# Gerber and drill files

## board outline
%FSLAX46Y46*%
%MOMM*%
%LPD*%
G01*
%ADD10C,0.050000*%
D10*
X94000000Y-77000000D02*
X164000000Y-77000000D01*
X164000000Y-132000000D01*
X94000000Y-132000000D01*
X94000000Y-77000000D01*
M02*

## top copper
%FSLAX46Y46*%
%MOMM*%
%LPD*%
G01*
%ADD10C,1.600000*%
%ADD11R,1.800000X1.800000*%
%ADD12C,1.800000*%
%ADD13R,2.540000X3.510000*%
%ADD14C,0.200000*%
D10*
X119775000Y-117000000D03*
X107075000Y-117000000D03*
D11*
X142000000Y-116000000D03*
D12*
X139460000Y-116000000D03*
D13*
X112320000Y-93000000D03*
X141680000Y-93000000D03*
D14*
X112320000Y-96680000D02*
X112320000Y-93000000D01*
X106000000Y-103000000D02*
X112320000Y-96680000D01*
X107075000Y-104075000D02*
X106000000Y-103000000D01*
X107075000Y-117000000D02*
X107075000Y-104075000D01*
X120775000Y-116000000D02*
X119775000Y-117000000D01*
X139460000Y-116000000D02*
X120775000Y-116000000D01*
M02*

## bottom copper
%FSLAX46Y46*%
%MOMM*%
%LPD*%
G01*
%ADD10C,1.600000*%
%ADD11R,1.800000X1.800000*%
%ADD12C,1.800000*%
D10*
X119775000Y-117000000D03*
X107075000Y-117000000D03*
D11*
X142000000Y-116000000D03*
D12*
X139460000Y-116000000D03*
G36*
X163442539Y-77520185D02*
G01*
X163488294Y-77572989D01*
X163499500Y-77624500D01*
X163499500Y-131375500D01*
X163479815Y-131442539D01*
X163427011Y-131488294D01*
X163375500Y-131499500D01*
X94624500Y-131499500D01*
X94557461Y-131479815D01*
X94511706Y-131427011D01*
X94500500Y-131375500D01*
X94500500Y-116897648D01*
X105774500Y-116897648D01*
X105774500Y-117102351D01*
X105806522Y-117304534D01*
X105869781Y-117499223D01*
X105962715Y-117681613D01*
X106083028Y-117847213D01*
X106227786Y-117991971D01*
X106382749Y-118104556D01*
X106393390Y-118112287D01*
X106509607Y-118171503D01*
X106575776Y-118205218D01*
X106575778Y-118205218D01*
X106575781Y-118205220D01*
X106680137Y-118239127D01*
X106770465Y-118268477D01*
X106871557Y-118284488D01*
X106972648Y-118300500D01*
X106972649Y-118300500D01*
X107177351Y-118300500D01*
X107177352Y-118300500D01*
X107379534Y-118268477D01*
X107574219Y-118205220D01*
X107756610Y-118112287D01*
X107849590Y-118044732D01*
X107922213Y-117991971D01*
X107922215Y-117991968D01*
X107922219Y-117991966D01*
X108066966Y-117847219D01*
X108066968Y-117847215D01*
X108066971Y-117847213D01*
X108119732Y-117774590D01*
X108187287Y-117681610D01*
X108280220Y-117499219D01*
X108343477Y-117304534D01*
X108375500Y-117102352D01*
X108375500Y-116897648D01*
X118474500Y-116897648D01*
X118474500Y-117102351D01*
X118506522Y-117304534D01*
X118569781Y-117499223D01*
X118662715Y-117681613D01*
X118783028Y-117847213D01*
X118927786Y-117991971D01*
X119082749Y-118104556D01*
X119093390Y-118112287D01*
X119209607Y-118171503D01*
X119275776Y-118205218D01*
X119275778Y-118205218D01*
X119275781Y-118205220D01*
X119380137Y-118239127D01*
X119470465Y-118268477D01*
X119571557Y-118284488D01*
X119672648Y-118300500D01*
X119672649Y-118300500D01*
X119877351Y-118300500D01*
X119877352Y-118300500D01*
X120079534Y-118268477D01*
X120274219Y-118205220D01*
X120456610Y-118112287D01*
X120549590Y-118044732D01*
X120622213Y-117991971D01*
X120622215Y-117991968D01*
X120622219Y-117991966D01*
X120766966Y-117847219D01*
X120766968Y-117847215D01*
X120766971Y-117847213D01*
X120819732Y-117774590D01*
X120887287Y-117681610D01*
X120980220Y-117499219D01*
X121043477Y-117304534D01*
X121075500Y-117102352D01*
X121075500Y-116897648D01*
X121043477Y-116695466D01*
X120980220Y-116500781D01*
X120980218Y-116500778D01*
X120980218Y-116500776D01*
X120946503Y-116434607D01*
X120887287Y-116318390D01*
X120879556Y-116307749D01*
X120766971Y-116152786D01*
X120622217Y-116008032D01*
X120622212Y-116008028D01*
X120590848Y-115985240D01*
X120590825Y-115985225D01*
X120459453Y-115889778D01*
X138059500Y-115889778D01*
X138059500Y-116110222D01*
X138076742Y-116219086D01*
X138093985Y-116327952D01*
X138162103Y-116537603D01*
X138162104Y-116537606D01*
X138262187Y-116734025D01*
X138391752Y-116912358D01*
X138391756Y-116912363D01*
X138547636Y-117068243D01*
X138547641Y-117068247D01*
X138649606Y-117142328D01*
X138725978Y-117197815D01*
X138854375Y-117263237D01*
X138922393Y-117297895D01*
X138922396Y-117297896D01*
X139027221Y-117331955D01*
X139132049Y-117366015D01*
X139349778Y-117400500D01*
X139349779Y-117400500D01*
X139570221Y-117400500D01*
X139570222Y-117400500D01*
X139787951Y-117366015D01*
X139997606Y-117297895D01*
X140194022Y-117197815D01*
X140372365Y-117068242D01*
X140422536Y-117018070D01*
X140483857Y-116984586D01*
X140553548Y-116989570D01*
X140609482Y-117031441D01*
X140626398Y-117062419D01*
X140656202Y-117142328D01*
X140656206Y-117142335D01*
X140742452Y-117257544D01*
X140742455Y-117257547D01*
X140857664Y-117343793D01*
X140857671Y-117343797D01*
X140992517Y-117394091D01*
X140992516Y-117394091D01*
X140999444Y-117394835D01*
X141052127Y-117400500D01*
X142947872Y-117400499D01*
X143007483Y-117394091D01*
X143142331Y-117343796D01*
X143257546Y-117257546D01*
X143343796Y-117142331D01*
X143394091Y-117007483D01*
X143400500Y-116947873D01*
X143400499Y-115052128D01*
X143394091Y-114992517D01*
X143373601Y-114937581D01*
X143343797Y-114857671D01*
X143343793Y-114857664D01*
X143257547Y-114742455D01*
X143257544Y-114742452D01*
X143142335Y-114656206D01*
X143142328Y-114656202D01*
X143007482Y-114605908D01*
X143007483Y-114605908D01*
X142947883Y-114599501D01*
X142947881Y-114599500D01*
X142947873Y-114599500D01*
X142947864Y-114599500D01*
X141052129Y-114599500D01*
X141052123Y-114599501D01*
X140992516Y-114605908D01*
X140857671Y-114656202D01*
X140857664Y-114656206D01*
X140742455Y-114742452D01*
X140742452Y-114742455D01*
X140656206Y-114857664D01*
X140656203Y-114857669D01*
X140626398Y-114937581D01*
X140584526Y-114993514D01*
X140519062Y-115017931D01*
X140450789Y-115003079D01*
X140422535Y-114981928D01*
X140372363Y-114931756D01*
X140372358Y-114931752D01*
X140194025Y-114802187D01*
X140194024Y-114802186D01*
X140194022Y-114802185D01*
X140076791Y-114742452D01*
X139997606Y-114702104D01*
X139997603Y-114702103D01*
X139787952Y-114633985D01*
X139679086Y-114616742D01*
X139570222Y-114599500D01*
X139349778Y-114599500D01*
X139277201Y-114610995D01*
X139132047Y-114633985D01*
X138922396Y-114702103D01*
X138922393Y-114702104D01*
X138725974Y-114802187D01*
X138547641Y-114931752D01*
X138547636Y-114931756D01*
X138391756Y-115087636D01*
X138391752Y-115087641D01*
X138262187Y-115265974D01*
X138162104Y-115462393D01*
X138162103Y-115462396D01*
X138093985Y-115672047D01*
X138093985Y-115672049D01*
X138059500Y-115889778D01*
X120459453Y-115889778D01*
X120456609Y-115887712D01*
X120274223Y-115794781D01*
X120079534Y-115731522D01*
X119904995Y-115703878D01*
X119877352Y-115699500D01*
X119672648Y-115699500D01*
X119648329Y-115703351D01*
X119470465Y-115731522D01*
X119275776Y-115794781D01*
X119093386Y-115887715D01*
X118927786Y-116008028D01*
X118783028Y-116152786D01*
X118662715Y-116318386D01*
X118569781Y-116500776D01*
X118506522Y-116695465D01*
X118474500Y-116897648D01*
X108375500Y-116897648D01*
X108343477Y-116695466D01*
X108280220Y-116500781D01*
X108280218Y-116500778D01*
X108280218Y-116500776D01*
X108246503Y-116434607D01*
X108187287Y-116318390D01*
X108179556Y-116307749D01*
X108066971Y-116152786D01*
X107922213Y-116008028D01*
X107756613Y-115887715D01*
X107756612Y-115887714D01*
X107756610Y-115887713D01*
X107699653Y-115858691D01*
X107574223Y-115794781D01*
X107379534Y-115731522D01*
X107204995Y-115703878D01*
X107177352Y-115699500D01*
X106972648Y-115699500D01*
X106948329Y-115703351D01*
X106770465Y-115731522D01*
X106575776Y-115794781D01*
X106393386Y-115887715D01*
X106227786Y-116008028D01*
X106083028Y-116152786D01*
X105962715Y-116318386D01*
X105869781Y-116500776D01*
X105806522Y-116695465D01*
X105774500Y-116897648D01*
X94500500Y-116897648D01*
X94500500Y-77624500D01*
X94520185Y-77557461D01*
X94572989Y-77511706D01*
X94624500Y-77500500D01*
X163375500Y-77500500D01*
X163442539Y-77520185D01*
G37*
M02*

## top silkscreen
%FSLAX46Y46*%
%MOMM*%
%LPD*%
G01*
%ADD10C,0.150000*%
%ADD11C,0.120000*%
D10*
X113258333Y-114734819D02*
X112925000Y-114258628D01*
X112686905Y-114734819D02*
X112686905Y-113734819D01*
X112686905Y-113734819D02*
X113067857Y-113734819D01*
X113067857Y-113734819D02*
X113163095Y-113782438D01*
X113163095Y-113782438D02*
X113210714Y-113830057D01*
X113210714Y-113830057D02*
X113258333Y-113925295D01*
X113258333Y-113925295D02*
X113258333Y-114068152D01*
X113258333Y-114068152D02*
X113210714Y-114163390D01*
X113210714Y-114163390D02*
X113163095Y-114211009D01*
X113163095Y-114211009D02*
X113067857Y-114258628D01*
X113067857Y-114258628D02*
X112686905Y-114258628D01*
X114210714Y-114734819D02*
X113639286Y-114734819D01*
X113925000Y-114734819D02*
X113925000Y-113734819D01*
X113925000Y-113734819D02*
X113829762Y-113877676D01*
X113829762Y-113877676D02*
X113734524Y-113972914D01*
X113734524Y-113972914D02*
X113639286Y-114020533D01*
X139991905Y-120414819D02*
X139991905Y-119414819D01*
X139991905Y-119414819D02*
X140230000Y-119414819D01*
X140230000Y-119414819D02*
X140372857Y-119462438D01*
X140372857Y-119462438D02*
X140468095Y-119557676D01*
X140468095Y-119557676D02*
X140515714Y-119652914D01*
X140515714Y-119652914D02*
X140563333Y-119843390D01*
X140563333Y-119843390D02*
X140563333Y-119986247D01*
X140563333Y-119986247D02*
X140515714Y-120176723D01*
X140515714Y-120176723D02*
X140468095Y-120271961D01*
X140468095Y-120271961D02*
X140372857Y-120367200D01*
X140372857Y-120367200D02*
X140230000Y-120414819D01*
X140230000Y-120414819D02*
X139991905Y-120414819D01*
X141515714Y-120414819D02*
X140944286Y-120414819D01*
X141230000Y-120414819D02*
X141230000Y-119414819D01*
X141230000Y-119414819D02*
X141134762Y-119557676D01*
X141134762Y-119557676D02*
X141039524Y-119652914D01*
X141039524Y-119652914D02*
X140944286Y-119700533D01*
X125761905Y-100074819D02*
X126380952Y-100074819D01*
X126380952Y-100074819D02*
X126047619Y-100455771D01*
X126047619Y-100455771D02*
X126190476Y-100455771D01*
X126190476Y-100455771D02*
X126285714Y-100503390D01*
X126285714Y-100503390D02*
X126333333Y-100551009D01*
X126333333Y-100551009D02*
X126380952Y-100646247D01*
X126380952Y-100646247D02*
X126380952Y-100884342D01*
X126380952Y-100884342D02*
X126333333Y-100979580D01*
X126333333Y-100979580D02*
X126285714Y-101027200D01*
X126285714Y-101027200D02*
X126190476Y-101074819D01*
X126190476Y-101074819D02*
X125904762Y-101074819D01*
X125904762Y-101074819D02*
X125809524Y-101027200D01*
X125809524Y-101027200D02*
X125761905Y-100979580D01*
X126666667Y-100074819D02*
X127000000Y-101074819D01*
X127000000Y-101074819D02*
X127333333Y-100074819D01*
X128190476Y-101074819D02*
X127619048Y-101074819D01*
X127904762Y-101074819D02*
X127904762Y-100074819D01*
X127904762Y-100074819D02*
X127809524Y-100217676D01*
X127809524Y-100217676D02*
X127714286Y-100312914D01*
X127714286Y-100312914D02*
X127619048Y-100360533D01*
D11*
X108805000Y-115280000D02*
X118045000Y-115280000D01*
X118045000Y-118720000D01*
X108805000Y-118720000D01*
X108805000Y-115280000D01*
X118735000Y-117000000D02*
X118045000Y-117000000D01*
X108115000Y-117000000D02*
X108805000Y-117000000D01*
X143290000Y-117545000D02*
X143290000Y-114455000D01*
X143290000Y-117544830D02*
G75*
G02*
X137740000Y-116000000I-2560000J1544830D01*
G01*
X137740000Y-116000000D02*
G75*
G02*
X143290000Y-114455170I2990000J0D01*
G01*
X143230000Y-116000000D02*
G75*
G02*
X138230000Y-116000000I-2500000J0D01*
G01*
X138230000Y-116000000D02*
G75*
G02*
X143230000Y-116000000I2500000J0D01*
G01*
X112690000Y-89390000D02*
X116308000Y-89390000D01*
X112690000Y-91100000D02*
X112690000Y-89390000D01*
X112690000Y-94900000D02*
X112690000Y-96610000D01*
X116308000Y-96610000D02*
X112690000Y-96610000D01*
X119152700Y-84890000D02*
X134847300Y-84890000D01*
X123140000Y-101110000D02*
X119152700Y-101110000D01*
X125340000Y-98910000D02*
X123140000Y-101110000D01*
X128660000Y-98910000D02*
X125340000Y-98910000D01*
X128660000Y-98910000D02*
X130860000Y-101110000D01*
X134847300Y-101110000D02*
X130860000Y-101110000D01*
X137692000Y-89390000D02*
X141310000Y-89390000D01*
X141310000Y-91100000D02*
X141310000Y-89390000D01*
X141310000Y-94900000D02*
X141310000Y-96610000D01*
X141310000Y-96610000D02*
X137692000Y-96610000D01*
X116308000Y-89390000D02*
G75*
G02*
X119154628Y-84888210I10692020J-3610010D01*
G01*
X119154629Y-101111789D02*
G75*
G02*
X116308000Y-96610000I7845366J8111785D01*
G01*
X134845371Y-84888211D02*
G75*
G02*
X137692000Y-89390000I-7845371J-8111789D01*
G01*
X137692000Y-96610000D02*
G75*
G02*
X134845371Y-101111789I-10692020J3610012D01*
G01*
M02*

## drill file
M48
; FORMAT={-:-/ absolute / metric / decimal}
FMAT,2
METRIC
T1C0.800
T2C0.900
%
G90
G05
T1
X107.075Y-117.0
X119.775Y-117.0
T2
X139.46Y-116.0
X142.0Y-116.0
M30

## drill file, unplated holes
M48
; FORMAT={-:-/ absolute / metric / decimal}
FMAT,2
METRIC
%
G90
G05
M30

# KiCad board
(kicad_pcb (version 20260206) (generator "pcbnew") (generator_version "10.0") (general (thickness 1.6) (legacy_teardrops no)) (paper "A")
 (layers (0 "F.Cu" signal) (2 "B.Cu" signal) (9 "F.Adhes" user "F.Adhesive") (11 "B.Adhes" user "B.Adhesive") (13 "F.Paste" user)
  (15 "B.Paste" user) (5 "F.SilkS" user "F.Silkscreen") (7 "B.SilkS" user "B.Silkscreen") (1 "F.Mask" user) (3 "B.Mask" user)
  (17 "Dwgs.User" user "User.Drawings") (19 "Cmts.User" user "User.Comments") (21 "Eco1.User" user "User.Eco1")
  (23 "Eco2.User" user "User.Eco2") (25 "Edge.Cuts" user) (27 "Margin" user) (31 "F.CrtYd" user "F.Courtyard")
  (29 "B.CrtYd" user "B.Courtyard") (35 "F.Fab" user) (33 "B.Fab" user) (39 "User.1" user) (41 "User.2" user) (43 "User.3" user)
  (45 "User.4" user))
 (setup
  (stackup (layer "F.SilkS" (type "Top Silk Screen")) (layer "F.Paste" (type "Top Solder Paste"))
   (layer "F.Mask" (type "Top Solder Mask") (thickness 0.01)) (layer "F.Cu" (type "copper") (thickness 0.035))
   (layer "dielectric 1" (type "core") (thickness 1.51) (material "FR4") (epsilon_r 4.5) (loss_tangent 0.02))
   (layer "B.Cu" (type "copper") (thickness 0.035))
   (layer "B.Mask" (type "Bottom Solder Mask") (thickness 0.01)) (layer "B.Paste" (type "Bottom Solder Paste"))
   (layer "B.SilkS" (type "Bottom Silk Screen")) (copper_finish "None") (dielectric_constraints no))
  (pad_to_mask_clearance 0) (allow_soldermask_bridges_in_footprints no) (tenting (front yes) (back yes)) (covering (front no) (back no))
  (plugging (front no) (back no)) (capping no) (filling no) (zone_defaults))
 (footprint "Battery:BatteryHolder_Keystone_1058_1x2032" (layer "F.Cu") (at 127 93)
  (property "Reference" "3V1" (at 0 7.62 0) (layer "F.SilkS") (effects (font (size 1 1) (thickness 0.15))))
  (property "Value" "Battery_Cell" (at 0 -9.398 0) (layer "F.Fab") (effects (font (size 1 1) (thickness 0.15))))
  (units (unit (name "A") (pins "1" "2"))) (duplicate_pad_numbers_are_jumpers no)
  (fp_line (start -14.31 -3.61) (end -10.692 -3.61) (stroke (width 0.12) (type solid)) (layer "F.SilkS"))
  (fp_line (start -14.31 -1.9) (end -14.31 -3.61) (stroke (width 0.12) (type solid)) (layer "F.SilkS"))
  (fp_line (start -14.31 1.9) (end -14.31 3.61) (stroke (width 0.12) (type solid)) (layer "F.SilkS"))
  (fp_line (start -10.692 3.61) (end -14.31 3.61) (stroke (width 0.12) (type solid)) (layer "F.SilkS"))
  (fp_line (start -7.8473 -8.11) (end 7.8473 -8.11) (stroke (width 0.12) (type solid)) (layer "F.SilkS"))
  (fp_line (start -3.86 8.11) (end -7.8473 8.11) (stroke (width 0.12) (type solid)) (layer "F.SilkS"))
  (fp_line (start -1.66 5.91) (end -3.86 8.11) (stroke (width 0.12) (type solid)) (layer "F.SilkS"))
  (fp_line (start 1.66 5.91) (end -1.66 5.91) (stroke (width 0.12) (type solid)) (layer "F.SilkS"))
  (fp_line (start 1.66 5.91) (end 3.86 8.11) (stroke (width 0.12) (type solid)) (layer "F.SilkS"))
  (fp_line (start 7.8473 8.11) (end 3.86 8.11) (stroke (width 0.12) (type solid)) (layer "F.SilkS"))
  (fp_line (start 10.692 -3.61) (end 14.31 -3.61) (stroke (width 0.12) (type solid)) (layer "F.SilkS"))
  (fp_line (start 14.31 -1.9) (end 14.31 -3.61) (stroke (width 0.12) (type solid)) (layer "F.SilkS"))
  (fp_line (start 14.31 1.9) (end 14.31 3.61) (stroke (width 0.12) (type solid)) (layer "F.SilkS"))
  (fp_line (start 14.31 3.61) (end 10.692 3.61) (stroke (width 0.12) (type solid)) (layer "F.SilkS"))
  (fp_arc (start -10.692 -3.61) (mid -9.538084 -6.031244) (end -7.845371 -8.111789) (stroke (width 0.12) (type solid)) (layer "F.SilkS"))
  (fp_arc (start -7.845371 8.111789) (mid -9.538085 6.031244) (end -10.692 3.61) (stroke (width 0.12) (type solid)) (layer "F.SilkS"))
  (fp_arc (start 7.845371 -8.111789) (mid 9.538085 -6.031244) (end 10.692 -3.61) (stroke (width 0.12) (type solid)) (layer "F.SilkS"))
  (fp_arc (start 10.692 3.61) (mid 9.538084 6.031244) (end 7.845371 8.111789) (stroke (width 0.12) (type solid)) (layer "F.SilkS"))
  (pad "1" smd rect (at -14.68 0) (size 2.54 3.51) (layers "F.Cu" "F.Mask" "F.Paste") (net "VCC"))
  (pad "2" smd rect (at 14.68 0) (size 2.54 3.51) (layers "F.Cu" "F.Mask" "F.Paste") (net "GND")))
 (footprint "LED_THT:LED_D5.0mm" (layer "F.Cu") (at 142 116 180)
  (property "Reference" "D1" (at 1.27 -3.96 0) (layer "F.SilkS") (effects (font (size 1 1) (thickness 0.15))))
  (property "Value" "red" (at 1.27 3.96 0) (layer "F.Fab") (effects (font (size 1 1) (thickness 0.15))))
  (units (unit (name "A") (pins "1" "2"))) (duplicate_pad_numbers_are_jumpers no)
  (fp_line (start -1.29 -1.545) (end -1.29 1.545) (stroke (width 0.12) (type solid)) (layer "F.SilkS"))
  (fp_arc (start 4.26 0) (mid 2.071779 2.880495) (end -1.29 1.54483) (stroke (width 0.12) (type solid)) (layer "F.SilkS"))
  (fp_arc (start -1.29 -1.54483) (mid 2.071779 -2.880495) (end 4.26 0) (stroke (width 0.12) (type solid)) (layer "F.SilkS"))
  (fp_circle (center 1.27 0) (end 3.77 0) (stroke (width 0.12) (type solid)) (fill no) (layer "F.SilkS"))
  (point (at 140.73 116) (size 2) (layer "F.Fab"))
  (pad "1" thru_hole rect (at 0 0 180) (size 1.8 1.8) (drill 0.9) (layers "*.Cu" "*.Mask") (remove_unused_layers no) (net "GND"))
  (pad "2" thru_hole circle (at 2.54 0 180) (size 1.8 1.8) (drill 0.9) (layers "*.Cu" "*.Mask") (remove_unused_layers no) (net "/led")))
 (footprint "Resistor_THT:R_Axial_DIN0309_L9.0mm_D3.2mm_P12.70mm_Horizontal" (layer "F.Cu") (at 107.075 117)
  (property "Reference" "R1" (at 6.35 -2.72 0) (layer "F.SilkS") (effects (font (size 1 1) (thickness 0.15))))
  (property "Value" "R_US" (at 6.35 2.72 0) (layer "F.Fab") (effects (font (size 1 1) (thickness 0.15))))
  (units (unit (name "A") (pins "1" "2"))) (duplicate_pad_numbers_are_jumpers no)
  (fp_line (start 1.04 0) (end 1.73 0) (stroke (width 0.12) (type solid)) (layer "F.SilkS"))
  (fp_line (start 11.66 0) (end 10.97 0) (stroke (width 0.12) (type solid)) (layer "F.SilkS"))
  (fp_rect (start 1.73 -1.72) (end 10.97 1.72) (stroke (width 0.12) (type solid)) (fill no) (layer "F.SilkS"))
  (pad "1" thru_hole circle (at 0 0) (size 1.6 1.6) (drill 0.8) (layers "*.Cu" "*.Mask") (remove_unused_layers no) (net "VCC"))
  (pad "2" thru_hole circle (at 12.7 0) (size 1.6 1.6) (drill 0.8) (layers "*.Cu" "*.Mask") (remove_unused_layers no) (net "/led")))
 (gr_rect (start 94 77) (end 164 132) (stroke (width 0.05) (type default)) (fill no) (layer "Edge.Cuts"))
 (segment (start 106 103) (end 112.32 96.68) (width 0.2) (layer "F.Cu") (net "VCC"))
 (segment (start 107.075 117) (end 107.075 104.075) (width 0.2) (layer "F.Cu") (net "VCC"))
 (segment (start 112.32 96.68) (end 112.32 93) (width 0.2) (layer "F.Cu") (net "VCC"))
 (segment (start 107.075 104.075) (end 106 103) (width 0.2) (layer "F.Cu") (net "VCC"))
 (segment (start 139.46 116) (end 120.775 116) (width 0.2) (layer "F.Cu") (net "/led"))
 (segment (start 120.775 116) (end 119.775 117) (width 0.2) (layer "F.Cu") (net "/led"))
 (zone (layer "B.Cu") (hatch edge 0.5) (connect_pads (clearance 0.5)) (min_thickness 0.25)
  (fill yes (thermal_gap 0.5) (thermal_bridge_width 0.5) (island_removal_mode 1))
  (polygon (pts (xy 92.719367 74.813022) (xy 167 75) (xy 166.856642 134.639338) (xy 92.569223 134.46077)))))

